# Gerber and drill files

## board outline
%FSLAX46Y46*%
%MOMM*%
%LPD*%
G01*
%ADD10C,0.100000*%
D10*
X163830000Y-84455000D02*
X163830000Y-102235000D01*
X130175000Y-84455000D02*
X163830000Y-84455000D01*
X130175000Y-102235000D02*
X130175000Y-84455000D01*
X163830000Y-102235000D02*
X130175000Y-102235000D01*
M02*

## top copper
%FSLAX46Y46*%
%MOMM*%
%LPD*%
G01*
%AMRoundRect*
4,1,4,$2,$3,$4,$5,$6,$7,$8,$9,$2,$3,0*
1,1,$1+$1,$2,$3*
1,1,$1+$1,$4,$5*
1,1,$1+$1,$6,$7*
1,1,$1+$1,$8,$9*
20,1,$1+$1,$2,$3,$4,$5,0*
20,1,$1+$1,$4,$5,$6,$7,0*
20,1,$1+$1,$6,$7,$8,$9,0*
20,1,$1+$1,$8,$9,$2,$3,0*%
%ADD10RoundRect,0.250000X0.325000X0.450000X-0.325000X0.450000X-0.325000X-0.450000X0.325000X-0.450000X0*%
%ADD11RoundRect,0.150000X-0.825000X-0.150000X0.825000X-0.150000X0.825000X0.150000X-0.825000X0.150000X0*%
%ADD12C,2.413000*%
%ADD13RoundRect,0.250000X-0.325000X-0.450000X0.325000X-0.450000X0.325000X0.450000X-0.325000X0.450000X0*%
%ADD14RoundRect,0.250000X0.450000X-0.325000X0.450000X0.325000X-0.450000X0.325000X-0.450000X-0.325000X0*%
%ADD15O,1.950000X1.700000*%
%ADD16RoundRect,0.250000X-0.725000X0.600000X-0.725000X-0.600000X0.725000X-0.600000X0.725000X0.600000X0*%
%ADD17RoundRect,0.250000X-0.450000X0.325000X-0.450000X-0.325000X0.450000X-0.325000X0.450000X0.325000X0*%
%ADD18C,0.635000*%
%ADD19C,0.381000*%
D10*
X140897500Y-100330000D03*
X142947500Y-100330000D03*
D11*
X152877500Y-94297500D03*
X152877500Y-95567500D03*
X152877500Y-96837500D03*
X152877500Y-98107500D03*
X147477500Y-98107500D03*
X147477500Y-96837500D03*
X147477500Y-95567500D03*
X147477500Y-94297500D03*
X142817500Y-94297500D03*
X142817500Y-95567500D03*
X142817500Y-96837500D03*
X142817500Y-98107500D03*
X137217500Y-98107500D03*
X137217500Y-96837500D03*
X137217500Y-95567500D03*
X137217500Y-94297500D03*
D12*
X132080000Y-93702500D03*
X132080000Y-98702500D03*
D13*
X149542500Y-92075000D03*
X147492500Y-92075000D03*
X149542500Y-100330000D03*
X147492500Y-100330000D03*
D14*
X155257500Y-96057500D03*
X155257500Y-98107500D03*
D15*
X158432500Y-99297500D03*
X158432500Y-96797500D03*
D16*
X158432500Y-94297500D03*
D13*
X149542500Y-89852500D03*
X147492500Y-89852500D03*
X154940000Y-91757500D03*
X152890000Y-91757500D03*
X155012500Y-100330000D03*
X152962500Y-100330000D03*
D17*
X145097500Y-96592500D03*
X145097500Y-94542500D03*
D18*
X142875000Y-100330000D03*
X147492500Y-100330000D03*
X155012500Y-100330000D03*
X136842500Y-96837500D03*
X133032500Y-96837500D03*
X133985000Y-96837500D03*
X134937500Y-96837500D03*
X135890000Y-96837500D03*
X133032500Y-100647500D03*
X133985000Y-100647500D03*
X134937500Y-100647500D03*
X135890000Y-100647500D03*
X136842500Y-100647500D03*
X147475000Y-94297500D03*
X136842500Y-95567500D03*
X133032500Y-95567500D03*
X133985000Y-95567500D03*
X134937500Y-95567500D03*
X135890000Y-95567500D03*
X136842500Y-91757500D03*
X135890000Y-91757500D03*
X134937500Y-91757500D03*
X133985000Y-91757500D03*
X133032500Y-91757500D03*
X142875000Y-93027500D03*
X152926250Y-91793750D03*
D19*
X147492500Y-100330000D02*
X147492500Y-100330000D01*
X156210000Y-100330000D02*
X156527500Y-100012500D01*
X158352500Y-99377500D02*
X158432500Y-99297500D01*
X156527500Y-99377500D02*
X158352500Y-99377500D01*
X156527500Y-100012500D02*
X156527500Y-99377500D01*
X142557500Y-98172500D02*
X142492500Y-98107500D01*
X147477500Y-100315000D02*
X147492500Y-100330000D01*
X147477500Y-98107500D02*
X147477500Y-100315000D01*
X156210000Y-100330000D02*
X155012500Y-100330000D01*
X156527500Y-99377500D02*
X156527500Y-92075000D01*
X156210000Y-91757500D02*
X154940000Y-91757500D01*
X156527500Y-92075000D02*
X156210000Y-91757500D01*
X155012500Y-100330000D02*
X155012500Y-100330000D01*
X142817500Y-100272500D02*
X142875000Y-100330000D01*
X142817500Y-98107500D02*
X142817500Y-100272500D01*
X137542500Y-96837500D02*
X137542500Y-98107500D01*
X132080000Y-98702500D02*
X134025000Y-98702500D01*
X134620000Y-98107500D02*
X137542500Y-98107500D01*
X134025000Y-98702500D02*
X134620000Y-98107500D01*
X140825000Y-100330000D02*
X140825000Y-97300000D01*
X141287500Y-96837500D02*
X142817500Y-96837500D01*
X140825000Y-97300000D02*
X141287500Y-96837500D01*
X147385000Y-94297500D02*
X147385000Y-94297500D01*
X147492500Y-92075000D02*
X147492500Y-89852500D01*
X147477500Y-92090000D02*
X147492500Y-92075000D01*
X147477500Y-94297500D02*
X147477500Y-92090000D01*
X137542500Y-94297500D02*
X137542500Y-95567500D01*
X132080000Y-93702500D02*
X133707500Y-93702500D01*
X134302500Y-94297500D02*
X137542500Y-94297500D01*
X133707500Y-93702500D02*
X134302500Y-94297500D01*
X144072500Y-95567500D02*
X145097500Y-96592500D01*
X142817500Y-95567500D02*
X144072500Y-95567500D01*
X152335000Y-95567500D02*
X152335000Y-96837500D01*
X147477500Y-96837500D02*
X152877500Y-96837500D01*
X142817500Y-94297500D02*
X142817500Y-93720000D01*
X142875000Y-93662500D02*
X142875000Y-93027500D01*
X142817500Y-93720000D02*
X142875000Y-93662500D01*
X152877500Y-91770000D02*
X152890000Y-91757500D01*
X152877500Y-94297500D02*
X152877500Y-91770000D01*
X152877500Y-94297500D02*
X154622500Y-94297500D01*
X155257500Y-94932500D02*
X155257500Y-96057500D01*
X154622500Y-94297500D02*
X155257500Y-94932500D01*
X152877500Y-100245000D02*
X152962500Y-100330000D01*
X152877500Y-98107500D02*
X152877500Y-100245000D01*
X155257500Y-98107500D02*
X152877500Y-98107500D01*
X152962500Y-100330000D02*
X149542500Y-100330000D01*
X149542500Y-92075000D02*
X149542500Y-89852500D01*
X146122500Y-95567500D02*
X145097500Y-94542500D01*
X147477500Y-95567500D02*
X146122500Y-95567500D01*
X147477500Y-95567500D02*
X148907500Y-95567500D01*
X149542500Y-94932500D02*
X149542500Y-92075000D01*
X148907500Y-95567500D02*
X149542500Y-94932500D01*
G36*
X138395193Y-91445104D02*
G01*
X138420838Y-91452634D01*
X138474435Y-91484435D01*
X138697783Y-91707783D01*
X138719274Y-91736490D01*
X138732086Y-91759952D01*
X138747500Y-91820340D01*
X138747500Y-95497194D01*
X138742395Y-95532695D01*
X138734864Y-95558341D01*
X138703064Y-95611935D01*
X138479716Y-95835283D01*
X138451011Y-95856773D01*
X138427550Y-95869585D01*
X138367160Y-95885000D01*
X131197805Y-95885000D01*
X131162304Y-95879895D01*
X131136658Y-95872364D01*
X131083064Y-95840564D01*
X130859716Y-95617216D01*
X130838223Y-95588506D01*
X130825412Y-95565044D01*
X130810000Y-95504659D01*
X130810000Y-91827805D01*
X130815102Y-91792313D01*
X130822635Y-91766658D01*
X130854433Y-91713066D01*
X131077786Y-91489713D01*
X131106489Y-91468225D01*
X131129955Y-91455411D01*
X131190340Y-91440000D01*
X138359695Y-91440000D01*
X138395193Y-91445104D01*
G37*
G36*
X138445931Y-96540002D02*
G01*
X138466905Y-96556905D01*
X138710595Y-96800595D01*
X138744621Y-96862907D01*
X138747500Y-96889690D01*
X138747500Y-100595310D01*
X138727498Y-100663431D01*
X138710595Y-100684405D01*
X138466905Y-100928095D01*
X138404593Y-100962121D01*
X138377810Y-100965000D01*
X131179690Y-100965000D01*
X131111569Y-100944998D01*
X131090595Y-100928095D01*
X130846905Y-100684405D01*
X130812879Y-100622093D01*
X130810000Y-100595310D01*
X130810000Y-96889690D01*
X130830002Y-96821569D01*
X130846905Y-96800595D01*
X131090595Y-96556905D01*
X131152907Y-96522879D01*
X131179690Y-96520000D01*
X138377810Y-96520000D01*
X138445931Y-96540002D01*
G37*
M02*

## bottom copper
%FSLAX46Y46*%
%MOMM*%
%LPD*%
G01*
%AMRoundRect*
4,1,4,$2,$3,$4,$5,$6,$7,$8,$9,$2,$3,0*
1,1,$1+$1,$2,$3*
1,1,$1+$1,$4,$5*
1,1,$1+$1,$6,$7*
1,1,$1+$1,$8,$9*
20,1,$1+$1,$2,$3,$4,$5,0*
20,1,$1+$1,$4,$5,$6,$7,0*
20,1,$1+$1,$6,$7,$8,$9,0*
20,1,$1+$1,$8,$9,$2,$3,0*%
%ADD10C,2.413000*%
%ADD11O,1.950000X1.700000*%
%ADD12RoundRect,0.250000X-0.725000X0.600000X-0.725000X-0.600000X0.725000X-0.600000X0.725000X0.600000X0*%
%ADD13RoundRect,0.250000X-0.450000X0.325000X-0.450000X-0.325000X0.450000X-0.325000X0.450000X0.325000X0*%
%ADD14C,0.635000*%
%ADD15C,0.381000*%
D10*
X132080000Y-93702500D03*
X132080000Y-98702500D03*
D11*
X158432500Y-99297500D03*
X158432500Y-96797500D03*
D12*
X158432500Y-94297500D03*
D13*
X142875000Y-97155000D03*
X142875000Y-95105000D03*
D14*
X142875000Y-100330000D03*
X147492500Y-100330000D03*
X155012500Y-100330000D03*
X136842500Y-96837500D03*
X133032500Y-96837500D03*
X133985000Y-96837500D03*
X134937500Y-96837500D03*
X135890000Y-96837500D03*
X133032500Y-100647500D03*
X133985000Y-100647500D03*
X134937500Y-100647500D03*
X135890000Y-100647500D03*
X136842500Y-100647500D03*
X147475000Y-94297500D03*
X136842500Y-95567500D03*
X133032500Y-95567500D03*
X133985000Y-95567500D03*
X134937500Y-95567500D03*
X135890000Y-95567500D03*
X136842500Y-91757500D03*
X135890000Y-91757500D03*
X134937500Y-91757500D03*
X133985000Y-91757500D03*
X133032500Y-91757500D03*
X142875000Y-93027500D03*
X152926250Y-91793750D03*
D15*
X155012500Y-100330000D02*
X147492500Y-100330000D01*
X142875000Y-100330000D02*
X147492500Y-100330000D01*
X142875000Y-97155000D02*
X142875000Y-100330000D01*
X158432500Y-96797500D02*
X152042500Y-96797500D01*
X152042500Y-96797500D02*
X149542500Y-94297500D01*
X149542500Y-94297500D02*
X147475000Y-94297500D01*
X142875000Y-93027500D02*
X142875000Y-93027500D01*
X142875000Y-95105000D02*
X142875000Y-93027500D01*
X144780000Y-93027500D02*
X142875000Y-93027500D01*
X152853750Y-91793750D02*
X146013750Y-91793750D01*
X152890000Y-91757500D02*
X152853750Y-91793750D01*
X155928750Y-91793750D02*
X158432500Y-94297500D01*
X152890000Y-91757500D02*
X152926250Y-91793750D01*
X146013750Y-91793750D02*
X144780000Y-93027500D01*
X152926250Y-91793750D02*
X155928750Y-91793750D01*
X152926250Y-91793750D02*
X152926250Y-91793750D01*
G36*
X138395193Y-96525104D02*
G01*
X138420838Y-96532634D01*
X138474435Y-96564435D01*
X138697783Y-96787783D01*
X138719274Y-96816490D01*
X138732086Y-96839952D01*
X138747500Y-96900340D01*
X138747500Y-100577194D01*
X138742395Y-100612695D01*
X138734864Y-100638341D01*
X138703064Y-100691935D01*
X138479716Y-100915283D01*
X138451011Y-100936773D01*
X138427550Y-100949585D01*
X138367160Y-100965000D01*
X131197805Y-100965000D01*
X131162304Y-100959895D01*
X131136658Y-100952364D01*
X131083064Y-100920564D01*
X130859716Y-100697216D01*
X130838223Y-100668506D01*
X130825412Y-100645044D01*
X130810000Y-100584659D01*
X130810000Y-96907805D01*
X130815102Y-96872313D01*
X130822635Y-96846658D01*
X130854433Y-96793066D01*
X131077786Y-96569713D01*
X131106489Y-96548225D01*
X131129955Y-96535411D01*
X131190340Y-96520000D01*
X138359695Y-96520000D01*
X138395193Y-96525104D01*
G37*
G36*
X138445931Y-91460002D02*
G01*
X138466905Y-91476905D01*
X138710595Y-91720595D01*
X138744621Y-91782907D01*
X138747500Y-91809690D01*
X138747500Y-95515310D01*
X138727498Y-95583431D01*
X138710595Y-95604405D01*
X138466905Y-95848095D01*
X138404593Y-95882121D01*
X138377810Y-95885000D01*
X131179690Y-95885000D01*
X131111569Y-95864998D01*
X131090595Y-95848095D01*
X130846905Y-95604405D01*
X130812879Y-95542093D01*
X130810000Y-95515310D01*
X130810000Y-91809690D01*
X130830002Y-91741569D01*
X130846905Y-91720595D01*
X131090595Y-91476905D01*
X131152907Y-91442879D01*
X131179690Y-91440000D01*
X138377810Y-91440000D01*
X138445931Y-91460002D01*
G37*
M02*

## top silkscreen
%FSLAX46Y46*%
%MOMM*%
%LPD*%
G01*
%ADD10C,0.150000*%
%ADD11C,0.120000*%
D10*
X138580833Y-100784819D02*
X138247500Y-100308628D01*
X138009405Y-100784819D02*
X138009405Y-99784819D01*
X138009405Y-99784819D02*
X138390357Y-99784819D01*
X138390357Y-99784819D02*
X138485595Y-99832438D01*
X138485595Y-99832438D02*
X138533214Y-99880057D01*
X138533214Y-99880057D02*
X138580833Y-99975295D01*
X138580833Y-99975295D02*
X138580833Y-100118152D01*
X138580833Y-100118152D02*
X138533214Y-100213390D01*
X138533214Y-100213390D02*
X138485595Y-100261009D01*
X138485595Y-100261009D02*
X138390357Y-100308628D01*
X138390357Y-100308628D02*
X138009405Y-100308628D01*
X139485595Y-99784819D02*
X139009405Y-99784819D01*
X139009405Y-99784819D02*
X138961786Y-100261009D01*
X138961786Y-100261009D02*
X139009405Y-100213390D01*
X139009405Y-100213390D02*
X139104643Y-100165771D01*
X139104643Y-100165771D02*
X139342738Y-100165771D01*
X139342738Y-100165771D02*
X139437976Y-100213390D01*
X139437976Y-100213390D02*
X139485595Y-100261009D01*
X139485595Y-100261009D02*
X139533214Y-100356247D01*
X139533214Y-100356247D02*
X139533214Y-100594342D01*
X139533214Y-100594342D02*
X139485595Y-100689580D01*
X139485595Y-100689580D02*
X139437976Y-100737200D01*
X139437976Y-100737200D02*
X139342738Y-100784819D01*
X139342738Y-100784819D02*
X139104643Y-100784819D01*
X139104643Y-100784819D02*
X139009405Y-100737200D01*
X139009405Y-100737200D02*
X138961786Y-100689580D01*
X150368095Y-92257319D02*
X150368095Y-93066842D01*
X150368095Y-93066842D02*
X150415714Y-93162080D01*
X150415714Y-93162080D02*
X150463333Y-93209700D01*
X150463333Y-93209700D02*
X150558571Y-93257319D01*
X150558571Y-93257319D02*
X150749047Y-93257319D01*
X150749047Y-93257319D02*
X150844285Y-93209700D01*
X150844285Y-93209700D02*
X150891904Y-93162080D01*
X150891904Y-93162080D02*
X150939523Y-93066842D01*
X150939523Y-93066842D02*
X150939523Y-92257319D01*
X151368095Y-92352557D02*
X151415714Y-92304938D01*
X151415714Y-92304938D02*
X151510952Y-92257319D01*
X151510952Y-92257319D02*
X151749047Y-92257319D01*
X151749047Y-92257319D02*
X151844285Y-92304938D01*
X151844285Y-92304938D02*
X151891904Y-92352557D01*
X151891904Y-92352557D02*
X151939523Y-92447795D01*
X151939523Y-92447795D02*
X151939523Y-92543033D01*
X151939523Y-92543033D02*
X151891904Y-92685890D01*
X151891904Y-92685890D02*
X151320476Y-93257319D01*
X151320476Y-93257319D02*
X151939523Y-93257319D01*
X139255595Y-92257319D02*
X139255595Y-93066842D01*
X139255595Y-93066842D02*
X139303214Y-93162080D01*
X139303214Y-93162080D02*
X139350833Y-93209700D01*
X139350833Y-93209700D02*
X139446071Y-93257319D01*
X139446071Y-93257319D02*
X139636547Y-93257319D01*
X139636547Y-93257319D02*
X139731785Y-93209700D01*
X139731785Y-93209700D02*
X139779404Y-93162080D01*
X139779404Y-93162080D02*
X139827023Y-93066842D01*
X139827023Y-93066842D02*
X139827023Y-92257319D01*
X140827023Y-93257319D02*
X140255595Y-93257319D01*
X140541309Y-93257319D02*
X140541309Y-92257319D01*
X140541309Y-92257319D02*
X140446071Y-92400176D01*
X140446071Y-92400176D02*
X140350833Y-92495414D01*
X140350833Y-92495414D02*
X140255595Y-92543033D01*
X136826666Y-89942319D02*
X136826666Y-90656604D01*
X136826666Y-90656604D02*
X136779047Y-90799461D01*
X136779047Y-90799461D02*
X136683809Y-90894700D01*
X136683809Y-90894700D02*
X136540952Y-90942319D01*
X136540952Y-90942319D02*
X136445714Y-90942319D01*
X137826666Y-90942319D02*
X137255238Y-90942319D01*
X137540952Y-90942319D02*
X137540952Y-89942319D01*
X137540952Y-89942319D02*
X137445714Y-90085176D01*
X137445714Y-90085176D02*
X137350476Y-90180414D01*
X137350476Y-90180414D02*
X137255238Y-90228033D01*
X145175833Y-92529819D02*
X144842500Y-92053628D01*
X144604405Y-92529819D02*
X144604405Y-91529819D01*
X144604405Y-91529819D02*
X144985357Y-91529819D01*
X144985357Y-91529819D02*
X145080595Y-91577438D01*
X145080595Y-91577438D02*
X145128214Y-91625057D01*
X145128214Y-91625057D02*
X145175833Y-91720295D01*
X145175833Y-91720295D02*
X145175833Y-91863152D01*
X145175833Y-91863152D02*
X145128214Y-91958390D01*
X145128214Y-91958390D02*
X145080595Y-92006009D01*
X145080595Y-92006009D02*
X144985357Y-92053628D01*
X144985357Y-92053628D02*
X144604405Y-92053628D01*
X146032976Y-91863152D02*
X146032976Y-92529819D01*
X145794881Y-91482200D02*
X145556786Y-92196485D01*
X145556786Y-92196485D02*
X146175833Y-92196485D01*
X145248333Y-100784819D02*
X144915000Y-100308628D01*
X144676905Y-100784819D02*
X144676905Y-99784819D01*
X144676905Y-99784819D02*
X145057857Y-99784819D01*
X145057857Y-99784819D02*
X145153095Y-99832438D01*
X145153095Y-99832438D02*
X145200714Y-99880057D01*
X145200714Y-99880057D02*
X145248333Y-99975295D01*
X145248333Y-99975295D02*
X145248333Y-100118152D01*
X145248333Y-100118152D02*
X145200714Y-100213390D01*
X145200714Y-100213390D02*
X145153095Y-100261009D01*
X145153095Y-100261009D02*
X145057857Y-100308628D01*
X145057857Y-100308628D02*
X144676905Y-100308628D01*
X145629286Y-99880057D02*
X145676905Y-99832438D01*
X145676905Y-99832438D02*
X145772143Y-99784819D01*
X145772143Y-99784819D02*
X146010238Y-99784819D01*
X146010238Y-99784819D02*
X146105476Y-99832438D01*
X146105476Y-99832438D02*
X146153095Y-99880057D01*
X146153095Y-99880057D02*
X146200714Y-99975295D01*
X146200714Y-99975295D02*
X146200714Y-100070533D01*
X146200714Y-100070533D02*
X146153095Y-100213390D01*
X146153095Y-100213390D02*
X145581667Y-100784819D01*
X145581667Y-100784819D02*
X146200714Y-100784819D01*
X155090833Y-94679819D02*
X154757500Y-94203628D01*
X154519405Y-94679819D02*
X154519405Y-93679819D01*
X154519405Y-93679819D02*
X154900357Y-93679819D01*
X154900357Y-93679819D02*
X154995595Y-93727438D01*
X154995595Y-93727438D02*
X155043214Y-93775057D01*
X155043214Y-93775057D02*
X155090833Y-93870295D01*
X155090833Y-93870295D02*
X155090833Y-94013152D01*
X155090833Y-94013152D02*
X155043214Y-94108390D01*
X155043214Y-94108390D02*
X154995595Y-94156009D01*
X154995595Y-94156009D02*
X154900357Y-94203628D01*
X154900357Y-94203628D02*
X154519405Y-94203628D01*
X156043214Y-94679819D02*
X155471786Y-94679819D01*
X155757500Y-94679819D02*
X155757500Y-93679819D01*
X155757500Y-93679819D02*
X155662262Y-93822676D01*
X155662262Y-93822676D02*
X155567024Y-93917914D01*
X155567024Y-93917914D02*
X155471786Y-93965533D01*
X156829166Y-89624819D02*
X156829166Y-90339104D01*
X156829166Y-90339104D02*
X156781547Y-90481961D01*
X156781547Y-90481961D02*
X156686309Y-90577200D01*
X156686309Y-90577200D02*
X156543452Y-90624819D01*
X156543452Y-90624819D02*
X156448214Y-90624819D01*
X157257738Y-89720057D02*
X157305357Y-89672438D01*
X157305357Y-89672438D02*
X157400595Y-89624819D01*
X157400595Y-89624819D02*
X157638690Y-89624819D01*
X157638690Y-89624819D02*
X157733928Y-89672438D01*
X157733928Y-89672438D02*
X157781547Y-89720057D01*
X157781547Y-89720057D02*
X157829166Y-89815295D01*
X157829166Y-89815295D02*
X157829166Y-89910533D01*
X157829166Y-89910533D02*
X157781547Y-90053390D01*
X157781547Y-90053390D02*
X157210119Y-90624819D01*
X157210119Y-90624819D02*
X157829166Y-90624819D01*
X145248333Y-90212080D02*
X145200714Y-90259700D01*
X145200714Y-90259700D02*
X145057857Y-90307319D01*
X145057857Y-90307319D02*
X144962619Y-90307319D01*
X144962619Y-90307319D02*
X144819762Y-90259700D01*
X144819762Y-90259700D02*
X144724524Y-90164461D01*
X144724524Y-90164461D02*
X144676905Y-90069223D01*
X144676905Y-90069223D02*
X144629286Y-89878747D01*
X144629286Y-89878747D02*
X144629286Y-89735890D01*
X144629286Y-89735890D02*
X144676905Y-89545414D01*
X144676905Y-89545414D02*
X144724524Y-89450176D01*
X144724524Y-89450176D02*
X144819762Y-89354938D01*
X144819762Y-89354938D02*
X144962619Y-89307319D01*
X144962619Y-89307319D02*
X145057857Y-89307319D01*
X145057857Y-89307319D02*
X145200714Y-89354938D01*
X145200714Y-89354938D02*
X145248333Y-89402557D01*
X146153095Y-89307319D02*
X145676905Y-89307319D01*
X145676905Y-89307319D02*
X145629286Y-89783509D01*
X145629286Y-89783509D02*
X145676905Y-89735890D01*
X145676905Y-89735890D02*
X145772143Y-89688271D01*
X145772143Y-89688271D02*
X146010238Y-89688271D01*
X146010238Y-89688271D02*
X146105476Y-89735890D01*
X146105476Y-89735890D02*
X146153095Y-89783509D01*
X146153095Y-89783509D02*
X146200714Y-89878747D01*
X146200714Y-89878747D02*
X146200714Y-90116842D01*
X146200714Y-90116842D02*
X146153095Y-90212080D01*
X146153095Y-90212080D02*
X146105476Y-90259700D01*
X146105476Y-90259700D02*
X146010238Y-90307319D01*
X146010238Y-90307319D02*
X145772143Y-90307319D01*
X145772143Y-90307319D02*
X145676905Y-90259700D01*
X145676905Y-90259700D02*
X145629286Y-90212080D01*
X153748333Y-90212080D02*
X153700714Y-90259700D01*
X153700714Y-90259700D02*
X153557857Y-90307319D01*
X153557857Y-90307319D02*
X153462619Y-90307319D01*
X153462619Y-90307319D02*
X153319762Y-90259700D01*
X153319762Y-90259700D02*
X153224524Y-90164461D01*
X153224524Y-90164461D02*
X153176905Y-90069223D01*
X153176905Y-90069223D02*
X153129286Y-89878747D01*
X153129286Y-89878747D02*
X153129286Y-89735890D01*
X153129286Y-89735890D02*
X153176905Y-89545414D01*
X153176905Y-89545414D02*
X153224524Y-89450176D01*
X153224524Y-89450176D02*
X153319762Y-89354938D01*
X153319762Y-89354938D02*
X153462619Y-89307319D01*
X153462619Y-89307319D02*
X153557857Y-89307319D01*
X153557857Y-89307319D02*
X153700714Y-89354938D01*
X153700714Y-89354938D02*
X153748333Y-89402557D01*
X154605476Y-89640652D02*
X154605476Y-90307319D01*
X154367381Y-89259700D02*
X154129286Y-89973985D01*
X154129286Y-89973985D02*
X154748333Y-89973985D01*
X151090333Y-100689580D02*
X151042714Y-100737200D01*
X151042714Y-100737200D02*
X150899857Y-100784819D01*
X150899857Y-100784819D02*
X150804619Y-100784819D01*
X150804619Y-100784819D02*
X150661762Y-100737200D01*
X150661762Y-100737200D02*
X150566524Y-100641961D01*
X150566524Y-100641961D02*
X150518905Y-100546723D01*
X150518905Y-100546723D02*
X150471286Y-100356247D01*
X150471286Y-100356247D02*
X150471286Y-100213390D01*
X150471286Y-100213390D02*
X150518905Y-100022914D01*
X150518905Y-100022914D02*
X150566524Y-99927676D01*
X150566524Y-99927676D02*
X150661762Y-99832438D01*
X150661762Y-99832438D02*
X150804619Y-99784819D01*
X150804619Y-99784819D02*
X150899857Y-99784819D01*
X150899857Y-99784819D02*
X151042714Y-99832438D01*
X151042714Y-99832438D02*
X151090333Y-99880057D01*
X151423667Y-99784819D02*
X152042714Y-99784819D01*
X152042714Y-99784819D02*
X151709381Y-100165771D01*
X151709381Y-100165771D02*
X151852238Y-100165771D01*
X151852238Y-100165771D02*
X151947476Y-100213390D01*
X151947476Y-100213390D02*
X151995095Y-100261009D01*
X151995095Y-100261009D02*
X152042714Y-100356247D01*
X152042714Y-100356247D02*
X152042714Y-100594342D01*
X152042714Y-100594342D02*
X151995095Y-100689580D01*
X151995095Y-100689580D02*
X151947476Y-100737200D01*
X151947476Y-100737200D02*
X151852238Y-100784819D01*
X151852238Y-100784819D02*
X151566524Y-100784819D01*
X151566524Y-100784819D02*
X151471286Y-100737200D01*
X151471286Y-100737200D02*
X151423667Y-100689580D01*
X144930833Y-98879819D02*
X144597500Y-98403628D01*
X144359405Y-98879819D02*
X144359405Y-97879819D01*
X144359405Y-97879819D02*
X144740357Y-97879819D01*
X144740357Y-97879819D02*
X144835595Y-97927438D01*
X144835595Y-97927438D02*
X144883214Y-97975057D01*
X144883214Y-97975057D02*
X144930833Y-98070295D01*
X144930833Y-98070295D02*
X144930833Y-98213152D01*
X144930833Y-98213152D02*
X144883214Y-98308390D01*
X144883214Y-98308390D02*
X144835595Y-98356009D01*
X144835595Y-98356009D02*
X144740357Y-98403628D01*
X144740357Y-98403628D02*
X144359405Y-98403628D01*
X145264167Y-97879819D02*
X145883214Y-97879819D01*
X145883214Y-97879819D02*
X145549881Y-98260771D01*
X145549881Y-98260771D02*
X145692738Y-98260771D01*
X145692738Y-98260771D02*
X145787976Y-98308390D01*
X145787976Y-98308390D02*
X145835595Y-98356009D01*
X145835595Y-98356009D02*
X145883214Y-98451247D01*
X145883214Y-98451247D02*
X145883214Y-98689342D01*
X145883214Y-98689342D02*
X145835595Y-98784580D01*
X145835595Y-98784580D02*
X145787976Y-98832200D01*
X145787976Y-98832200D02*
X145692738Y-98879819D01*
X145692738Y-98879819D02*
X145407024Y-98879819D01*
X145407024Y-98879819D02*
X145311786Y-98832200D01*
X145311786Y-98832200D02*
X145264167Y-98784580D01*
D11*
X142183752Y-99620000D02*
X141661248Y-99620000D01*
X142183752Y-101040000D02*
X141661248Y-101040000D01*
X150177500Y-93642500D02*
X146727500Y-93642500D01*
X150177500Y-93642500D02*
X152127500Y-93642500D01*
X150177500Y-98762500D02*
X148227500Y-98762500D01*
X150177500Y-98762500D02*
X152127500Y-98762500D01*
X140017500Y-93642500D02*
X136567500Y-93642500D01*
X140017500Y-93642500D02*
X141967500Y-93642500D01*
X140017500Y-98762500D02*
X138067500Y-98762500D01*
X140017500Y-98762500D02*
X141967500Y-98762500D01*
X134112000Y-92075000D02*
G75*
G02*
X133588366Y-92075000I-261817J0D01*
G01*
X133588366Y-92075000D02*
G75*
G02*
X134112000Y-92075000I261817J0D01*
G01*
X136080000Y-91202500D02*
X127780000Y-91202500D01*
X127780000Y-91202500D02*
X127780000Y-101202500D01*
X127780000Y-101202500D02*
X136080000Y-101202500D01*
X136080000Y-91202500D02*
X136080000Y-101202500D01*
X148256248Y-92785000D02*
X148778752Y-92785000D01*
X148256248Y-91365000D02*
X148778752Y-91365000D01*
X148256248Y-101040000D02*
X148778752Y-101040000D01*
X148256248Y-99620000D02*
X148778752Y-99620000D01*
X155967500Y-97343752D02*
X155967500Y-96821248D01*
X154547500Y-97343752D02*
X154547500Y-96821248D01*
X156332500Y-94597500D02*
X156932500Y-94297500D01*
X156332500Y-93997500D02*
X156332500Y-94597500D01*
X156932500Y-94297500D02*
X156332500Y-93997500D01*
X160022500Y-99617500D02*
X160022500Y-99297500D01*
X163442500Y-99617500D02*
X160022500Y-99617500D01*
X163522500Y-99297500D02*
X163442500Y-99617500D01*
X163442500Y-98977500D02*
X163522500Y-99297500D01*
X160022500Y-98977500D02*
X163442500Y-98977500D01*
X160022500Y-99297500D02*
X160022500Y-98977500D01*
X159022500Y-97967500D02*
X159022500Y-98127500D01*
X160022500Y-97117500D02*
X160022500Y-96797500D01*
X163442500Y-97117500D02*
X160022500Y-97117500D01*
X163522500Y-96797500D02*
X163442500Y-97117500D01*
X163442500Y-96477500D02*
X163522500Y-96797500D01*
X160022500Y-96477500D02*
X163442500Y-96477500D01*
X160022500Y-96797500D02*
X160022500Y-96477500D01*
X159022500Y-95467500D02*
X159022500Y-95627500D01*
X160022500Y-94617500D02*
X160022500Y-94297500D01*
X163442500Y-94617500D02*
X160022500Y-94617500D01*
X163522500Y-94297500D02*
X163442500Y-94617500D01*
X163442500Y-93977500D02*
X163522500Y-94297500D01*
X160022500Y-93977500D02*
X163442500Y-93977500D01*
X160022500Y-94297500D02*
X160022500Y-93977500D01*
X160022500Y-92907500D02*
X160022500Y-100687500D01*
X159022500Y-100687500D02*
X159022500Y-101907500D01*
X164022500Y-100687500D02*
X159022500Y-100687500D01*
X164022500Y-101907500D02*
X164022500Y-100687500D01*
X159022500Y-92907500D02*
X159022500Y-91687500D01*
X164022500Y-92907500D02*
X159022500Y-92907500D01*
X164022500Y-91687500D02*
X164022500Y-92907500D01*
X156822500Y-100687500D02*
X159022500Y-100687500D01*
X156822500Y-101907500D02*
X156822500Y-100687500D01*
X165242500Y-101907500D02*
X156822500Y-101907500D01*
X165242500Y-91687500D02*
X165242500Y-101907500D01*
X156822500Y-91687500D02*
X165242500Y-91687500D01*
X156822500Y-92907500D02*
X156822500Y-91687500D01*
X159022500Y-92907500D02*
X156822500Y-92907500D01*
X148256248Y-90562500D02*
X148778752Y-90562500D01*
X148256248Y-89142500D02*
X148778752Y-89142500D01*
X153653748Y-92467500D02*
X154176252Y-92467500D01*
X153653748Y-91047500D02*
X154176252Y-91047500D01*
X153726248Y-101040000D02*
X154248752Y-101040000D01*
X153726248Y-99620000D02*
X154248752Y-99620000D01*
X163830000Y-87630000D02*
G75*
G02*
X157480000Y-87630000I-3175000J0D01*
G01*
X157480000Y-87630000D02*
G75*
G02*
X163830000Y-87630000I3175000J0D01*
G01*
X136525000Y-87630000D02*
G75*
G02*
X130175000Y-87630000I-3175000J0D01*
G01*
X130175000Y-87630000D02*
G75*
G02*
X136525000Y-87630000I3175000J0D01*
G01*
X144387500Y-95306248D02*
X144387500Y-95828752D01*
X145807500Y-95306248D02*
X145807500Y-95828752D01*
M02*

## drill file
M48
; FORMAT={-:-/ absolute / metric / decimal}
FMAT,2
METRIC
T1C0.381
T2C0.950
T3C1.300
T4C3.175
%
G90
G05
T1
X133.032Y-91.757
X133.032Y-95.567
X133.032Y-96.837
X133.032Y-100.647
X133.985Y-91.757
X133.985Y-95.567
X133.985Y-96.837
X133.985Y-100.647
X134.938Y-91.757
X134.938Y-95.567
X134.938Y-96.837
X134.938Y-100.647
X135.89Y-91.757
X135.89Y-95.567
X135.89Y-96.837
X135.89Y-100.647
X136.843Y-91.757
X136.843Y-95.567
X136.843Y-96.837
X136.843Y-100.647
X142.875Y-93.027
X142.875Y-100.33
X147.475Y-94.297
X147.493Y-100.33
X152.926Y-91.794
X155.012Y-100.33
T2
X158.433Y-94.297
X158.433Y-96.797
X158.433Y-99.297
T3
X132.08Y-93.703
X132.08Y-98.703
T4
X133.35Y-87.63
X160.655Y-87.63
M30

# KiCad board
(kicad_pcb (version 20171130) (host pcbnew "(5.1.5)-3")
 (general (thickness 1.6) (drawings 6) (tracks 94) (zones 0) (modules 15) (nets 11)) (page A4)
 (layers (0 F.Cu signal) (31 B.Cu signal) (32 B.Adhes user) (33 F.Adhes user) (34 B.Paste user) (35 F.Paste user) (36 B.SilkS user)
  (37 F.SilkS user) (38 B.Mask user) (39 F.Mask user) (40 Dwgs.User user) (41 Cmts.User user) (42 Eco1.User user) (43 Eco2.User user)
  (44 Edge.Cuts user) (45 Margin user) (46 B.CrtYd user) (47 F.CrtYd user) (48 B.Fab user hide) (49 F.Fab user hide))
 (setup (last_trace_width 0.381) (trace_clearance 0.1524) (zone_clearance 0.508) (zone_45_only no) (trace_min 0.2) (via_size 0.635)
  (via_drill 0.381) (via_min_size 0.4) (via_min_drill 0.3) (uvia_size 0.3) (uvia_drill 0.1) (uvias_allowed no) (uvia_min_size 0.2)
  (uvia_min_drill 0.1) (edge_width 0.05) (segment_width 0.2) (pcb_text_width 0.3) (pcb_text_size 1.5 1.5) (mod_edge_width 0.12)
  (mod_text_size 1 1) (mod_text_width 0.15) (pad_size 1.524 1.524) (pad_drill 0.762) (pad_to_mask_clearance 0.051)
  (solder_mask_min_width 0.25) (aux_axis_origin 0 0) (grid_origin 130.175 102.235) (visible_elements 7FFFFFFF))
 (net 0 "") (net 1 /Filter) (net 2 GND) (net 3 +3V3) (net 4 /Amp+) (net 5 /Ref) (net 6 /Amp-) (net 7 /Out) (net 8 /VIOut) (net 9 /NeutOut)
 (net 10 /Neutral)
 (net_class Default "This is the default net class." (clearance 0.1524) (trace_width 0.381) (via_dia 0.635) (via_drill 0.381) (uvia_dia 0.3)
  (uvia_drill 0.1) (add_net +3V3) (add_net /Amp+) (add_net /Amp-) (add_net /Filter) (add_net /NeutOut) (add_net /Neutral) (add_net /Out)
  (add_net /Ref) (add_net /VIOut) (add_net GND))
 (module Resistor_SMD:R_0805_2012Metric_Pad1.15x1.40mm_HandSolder (layer F.Cu) (at 141.9225 100.33 180)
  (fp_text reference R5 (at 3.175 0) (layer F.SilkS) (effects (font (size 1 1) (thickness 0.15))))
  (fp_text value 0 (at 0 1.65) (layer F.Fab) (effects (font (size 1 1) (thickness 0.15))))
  (fp_line (start -0.261252 0.71) (end 0.261252 0.71) (layer F.SilkS) (width 0.12))
  (fp_line (start -0.261252 -0.71) (end 0.261252 -0.71) (layer F.SilkS) (width 0.12))
  (pad 2 smd roundrect (at 1.025 0 180) (size 1.15 1.4) (layers F.Cu F.Paste F.Mask) (roundrect_rratio 0.217391) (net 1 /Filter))
  (pad 1 smd roundrect (at -1.025 0 180) (size 1.15 1.4) (layers F.Cu F.Paste F.Mask) (roundrect_rratio 0.217391) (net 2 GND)))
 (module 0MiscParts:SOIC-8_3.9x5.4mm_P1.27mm (layer F.Cu) (at 150.1775 96.2025)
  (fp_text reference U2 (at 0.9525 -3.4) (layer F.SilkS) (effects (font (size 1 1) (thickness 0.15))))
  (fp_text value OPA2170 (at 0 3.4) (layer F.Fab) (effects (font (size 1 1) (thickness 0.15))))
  (fp_line (start 0 -2.56) (end -3.45 -2.56) (layer F.SilkS) (width 0.12))
  (fp_line (start 0 -2.56) (end 1.95 -2.56) (layer F.SilkS) (width 0.12))
  (fp_line (start 0 2.56) (end -1.95 2.56) (layer F.SilkS) (width 0.12))
  (fp_line (start 0 2.56) (end 1.95 2.56) (layer F.SilkS) (width 0.12))
  (pad 8 smd roundrect (at 2.7 -1.905) (size 1.95 0.6) (layers F.Cu F.Paste F.Mask) (roundrect_rratio 0.25) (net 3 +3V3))
  (pad 7 smd roundrect (at 2.7 -0.635) (size 1.95 0.6) (layers F.Cu F.Paste F.Mask) (roundrect_rratio 0.25) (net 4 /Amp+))
  (pad 6 smd roundrect (at 2.7 0.635) (size 1.95 0.6) (layers F.Cu F.Paste F.Mask) (roundrect_rratio 0.25) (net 4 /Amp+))
  (pad 5 smd roundrect (at 2.7 1.905) (size 1.95 0.6) (layers F.Cu F.Paste F.Mask) (roundrect_rratio 0.25) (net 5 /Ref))
  (pad 4 smd roundrect (at -2.7 1.905) (size 1.95 0.6) (layers F.Cu F.Paste F.Mask) (roundrect_rratio 0.25) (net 2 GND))
  (pad 3 smd roundrect (at -2.7 0.635) (size 1.95 0.6) (layers F.Cu F.Paste F.Mask) (roundrect_rratio 0.25) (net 4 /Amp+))
  (pad 2 smd roundrect (at -2.7 -0.635) (size 1.95 0.6) (layers F.Cu F.Paste F.Mask) (roundrect_rratio 0.25) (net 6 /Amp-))
  (pad 1 smd roundrect (at -2.7 -1.905) (size 1.95 0.6) (layers F.Cu F.Paste F.Mask) (roundrect_rratio 0.25) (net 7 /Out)))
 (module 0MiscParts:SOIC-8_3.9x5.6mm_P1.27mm (layer F.Cu) (at 140.0175 96.2025)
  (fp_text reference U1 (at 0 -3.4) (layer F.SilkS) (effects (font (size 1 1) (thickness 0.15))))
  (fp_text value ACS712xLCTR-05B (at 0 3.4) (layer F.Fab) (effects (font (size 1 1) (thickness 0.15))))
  (fp_line (start 0 -2.56) (end -3.45 -2.56) (layer F.SilkS) (width 0.12))
  (fp_line (start 0 -2.56) (end 1.95 -2.56) (layer F.SilkS) (width 0.12))
  (fp_line (start 0 2.56) (end -1.95 2.56) (layer F.SilkS) (width 0.12))
  (fp_line (start 0 2.56) (end 1.95 2.56) (layer F.SilkS) (width 0.12))
  (pad 8 smd roundrect (at 2.8 -1.905) (size 1.95 0.6) (layers F.Cu F.Paste F.Mask) (roundrect_rratio 0.25) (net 3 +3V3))
  (pad 7 smd roundrect (at 2.8 -0.635) (size 1.95 0.6) (layers F.Cu F.Paste F.Mask) (roundrect_rratio 0.25) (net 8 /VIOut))
  (pad 6 smd roundrect (at 2.8 0.635) (size 1.95 0.6) (layers F.Cu F.Paste F.Mask) (roundrect_rratio 0.25) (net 1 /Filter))
  (pad 5 smd roundrect (at 2.8 1.905) (size 1.95 0.6) (layers F.Cu F.Paste F.Mask) (roundrect_rratio 0.25) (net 2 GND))
  (pad 4 smd roundrect (at -2.8 1.905) (size 1.95 0.6) (layers F.Cu F.Paste F.Mask) (roundrect_rratio 0.25) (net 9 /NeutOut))
  (pad 3 smd roundrect (at -2.8 0.635) (size 1.95 0.6) (layers F.Cu F.Paste F.Mask) (roundrect_rratio 0.25) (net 9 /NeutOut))
  (pad 2 smd roundrect (at -2.8 -0.635) (size 1.95 0.6) (layers F.Cu F.Paste F.Mask) (roundrect_rratio 0.25) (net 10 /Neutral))
  (pad 1 smd roundrect (at -2.8 -1.905) (size 1.95 0.6) (layers F.Cu F.Paste F.Mask) (roundrect_rratio 0.25) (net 10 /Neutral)))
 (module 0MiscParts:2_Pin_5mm (layer F.Cu) (at 132.08 96.2025 270)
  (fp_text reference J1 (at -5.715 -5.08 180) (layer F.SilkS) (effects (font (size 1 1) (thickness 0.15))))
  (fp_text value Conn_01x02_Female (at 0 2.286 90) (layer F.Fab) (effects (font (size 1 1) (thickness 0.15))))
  (fp_circle (center -4.1275 -1.770183) (end -4.064 -1.516183) (layer F.SilkS) (width 0.12))
  (fp_line (start -5 -4) (end -5 4.3) (layer F.SilkS) (width 0.12))
  (fp_line (start -5 4.3) (end 5 4.3) (layer F.SilkS) (width 0.12))
  (fp_line (start 5 4.3) (end 5 -4) (layer F.SilkS) (width 0.12))
  (fp_line (start -5 -4) (end 5 -4) (layer F.SilkS) (width 0.12))
  (pad 1 thru_hole circle (at -2.5 0 270) (size 2.413 2.413) (drill 1.3) (layers *.Cu *.Mask) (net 10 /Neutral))
  (pad 2 thru_hole circle (at 2.5 0 270) (size 2.413 2.413) (drill 1.3) (layers *.Cu *.Mask) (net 9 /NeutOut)))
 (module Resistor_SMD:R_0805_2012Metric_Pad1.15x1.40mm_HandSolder (layer F.Cu) (at 148.5175 92.075)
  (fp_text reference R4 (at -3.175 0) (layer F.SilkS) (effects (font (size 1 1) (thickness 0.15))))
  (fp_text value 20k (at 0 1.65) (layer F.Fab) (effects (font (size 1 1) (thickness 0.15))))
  (fp_line (start -0.261252 0.71) (end 0.261252 0.71) (layer F.SilkS) (width 0.12))
  (fp_line (start -0.261252 -0.71) (end 0.261252 -0.71) (layer F.SilkS) (width 0.12))
  (pad 2 smd roundrect (at 1.025 0) (size 1.15 1.4) (layers F.Cu F.Paste F.Mask) (roundrect_rratio 0.217391) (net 6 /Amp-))
  (pad 1 smd roundrect (at -1.025 0) (size 1.15 1.4) (layers F.Cu F.Paste F.Mask) (roundrect_rratio 0.217391) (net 7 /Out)))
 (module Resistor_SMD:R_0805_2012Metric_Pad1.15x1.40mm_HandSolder (layer F.Cu) (at 148.5175 100.33)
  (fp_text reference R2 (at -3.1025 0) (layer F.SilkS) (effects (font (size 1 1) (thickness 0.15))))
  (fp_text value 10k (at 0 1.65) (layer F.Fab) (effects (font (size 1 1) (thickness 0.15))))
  (fp_line (start -0.261252 0.71) (end 0.261252 0.71) (layer F.SilkS) (width 0.12))
  (fp_line (start -0.261252 -0.71) (end 0.261252 -0.71) (layer F.SilkS) (width 0.12))
  (pad 2 smd roundrect (at 1.025 0) (size 1.15 1.4) (layers F.Cu F.Paste F.Mask) (roundrect_rratio 0.217391) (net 5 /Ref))
  (pad 1 smd roundrect (at -1.025 0) (size 1.15 1.4) (layers F.Cu F.Paste F.Mask) (roundrect_rratio 0.217391) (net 2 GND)))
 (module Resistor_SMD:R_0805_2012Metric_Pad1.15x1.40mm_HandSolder (layer F.Cu) (at 155.2575 97.0825 90)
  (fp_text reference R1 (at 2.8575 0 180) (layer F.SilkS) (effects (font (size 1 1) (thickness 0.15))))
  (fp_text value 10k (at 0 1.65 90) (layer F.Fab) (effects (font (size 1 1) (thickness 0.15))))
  (fp_line (start -0.261252 0.71) (end 0.261252 0.71) (layer F.SilkS) (width 0.12))
  (fp_line (start -0.261252 -0.71) (end 0.261252 -0.71) (layer F.SilkS) (width 0.12))
  (pad 2 smd roundrect (at 1.025 0 90) (size 1.15 1.4) (layers F.Cu F.Paste F.Mask) (roundrect_rratio 0.217391) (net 3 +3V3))
  (pad 1 smd roundrect (at -1.025 0 90) (size 1.15 1.4) (layers F.Cu F.Paste F.Mask) (roundrect_rratio 0.217391) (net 5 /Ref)))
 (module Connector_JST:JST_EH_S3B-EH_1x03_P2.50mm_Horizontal (layer F.Cu) (at 158.4325 94.2975 270)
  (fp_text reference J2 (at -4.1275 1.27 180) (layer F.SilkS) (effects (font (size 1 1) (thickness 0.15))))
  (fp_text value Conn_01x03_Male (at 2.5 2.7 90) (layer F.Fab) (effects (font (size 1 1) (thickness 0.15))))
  (fp_line (start 0.3 2.1) (end 0 1.5) (layer F.SilkS) (width 0.12))
  (fp_line (start -0.3 2.1) (end 0.3 2.1) (layer F.SilkS) (width 0.12))
  (fp_line (start 0 1.5) (end -0.3 2.1) (layer F.SilkS) (width 0.12))
  (fp_line (start 5.32 -1.59) (end 5 -1.59) (layer F.SilkS) (width 0.12))
  (fp_line (start 5.32 -5.01) (end 5.32 -1.59) (layer F.SilkS) (width 0.12))
  (fp_line (start 5 -5.09) (end 5.32 -5.01) (layer F.SilkS) (width 0.12))
  (fp_line (start 4.68 -5.01) (end 5 -5.09) (layer F.SilkS) (width 0.12))
  (fp_line (start 4.68 -1.59) (end 4.68 -5.01) (layer F.SilkS) (width 0.12))
  (fp_line (start 5 -1.59) (end 4.68 -1.59) (layer F.SilkS) (width 0.12))
  (fp_line (start 3.67 -0.59) (end 3.83 -0.59) (layer F.SilkS) (width 0.12))
  (fp_line (start 2.82 -1.59) (end 2.5 -1.59) (layer F.SilkS) (width 0.12))
  (fp_line (start 2.82 -5.01) (end 2.82 -1.59) (layer F.SilkS) (width 0.12))
  (fp_line (start 2.5 -5.09) (end 2.82 -5.01) (layer F.SilkS) (width 0.12))
  (fp_line (start 2.18 -5.01) (end 2.5 -5.09) (layer F.SilkS) (width 0.12))
  (fp_line (start 2.18 -1.59) (end 2.18 -5.01) (layer F.SilkS) (width 0.12))
  (fp_line (start 2.5 -1.59) (end 2.18 -1.59) (layer F.SilkS) (width 0.12))
  (fp_line (start 1.17 -0.59) (end 1.33 -0.59) (layer F.SilkS) (width 0.12))
  (fp_line (start 0.32 -1.59) (end 0 -1.59) (layer F.SilkS) (width 0.12))
  (fp_line (start 0.32 -5.01) (end 0.32 -1.59) (layer F.SilkS) (width 0.12))
  (fp_line (start 0 -5.09) (end 0.32 -5.01) (layer F.SilkS) (width 0.12))
  (fp_line (start -0.32 -5.01) (end 0 -5.09) (layer F.SilkS) (width 0.12))
  (fp_line (start -0.32 -1.59) (end -0.32 -5.01) (layer F.SilkS) (width 0.12))
  (fp_line (start 0 -1.59) (end -0.32 -1.59) (layer F.SilkS) (width 0.12))
  (fp_line (start -1.39 -1.59) (end 6.39 -1.59) (layer F.SilkS) (width 0.12))
  (fp_line (start 6.39 -0.59) (end 7.61 -0.59) (layer F.SilkS) (width 0.12))
  (fp_line (start 6.39 -5.59) (end 6.39 -0.59) (layer F.SilkS) (width 0.12))
  (fp_line (start 7.61 -5.59) (end 6.39 -5.59) (layer F.SilkS) (width 0.12))
  (fp_line (start -1.39 -0.59) (end -2.61 -0.59) (layer F.SilkS) (width 0.12))
  (fp_line (start -1.39 -5.59) (end -1.39 -0.59) (layer F.SilkS) (width 0.12))
  (fp_line (start -2.61 -5.59) (end -1.39 -5.59) (layer F.SilkS) (width 0.12))
  (fp_line (start 6.39 1.61) (end 6.39 -0.59) (layer F.SilkS) (width 0.12))
  (fp_line (start 7.61 1.61) (end 6.39 1.61) (layer F.SilkS) (width 0.12))
  (fp_line (start 7.61 -6.81) (end 7.61 1.61) (layer F.SilkS) (width 0.12))
  (fp_line (start -2.61 -6.81) (end 7.61 -6.81) (layer F.SilkS) (width 0.12))
  (fp_line (start -2.61 1.61) (end -2.61 -6.81) (layer F.SilkS) (width 0.12))
  (fp_line (start -1.39 1.61) (end -2.61 1.61) (layer F.SilkS) (width 0.12))
  (fp_line (start -1.39 -0.59) (end -1.39 1.61) (layer F.SilkS) (width 0.12))
  (pad 3 thru_hole oval (at 5 0 270) (size 1.7 1.95) (drill 0.95) (layers *.Cu *.Mask) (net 2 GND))
  (pad 2 thru_hole oval (at 2.5 0 270) (size 1.7 1.95) (drill 0.95) (layers *.Cu *.Mask) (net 7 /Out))
  (pad 1 thru_hole roundrect (at 0 0 270) (size 1.7 1.95) (drill 0.95) (layers *.Cu *.Mask) (roundrect_rratio 0.147059) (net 3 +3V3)))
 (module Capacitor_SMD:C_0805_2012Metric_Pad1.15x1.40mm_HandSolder (layer F.Cu) (at 148.5175 89.8525)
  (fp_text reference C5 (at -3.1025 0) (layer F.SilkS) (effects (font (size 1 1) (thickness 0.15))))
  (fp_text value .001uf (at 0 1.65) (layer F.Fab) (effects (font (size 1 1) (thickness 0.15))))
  (fp_line (start -0.261252 0.71) (end 0.261252 0.71) (layer F.SilkS) (width 0.12))
  (fp_line (start -0.261252 -0.71) (end 0.261252 -0.71) (layer F.SilkS) (width 0.12))
  (pad 2 smd roundrect (at 1.025 0) (size 1.15 1.4) (layers F.Cu F.Paste F.Mask) (roundrect_rratio 0.217391) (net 6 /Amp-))
  (pad 1 smd roundrect (at -1.025 0) (size 1.15 1.4) (layers F.Cu F.Paste F.Mask) (roundrect_rratio 0.217391) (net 7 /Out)))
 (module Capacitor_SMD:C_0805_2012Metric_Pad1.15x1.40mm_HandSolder (layer F.Cu) (at 153.915 91.7575)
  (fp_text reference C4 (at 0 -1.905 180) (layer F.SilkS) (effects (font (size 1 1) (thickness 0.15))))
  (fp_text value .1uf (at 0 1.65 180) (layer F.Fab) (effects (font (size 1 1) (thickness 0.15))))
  (fp_line (start -0.261252 0.71) (end 0.261252 0.71) (layer F.SilkS) (width 0.12))
  (fp_line (start -0.261252 -0.71) (end 0.261252 -0.71) (layer F.SilkS) (width 0.12))
  (pad 2 smd roundrect (at 1.025 0) (size 1.15 1.4) (layers F.Cu F.Paste F.Mask) (roundrect_rratio 0.217391) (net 2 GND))
  (pad 1 smd roundrect (at -1.025 0) (size 1.15 1.4) (layers F.Cu F.Paste F.Mask) (roundrect_rratio 0.217391) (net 3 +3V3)))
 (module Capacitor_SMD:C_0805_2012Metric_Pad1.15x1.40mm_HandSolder (layer F.Cu) (at 153.9875 100.33)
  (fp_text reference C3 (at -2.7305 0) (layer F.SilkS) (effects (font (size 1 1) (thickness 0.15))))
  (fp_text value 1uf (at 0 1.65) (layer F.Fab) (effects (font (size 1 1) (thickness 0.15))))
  (fp_line (start -0.261252 0.71) (end 0.261252 0.71) (layer F.SilkS) (width 0.12))
  (fp_line (start -0.261252 -0.71) (end 0.261252 -0.71) (layer F.SilkS) (width 0.12))
  (pad 2 smd roundrect (at 1.025 0) (size 1.15 1.4) (layers F.Cu F.Paste F.Mask) (roundrect_rratio 0.217391) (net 2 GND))
  (pad 1 smd roundrect (at -1.025 0) (size 1.15 1.4) (layers F.Cu F.Paste F.Mask) (roundrect_rratio 0.217391) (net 5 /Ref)))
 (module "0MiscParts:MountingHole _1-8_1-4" (layer F.Cu) (at 160.655 87.63)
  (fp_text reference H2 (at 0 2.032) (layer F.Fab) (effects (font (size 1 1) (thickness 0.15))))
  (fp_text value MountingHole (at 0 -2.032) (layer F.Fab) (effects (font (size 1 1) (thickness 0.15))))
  (fp_circle (center 0 0) (end 3.175 0) (layer F.SilkS) (width 0.12))
  (pad "" np_thru_hole circle (at 0 0) (size 3.175 3.175) (drill 3.175) (layers *.Cu *.Mask)))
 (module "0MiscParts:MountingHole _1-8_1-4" (layer F.Cu) (at 133.35 87.63)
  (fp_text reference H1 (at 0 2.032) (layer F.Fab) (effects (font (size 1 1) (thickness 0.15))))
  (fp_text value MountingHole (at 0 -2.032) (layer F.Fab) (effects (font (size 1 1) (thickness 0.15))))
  (fp_circle (center 0 0) (end 3.175 0) (layer F.SilkS) (width 0.12))
  (pad "" np_thru_hole circle (at 0 0) (size 3.175 3.175) (drill 3.175) (layers *.Cu *.Mask)))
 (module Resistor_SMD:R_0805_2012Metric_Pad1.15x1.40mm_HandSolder (layer F.Cu) (at 145.0975 95.5675 270)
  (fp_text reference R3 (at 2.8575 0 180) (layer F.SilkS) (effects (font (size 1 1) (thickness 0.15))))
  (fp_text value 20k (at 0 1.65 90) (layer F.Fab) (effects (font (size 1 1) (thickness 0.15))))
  (fp_line (start -0.261252 0.71) (end 0.261252 0.71) (layer F.SilkS) (width 0.12))
  (fp_line (start -0.261252 -0.71) (end 0.261252 -0.71) (layer F.SilkS) (width 0.12))
  (pad 2 smd roundrect (at 1.025 0 270) (size 1.15 1.4) (layers F.Cu F.Paste F.Mask) (roundrect_rratio 0.217391) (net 8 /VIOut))
  (pad 1 smd roundrect (at -1.025 0 270) (size 1.15 1.4) (layers F.Cu F.Paste F.Mask) (roundrect_rratio 0.217391) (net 6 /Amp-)))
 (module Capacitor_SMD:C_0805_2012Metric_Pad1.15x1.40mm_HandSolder (layer B.Cu) (at 142.875 96.13 270)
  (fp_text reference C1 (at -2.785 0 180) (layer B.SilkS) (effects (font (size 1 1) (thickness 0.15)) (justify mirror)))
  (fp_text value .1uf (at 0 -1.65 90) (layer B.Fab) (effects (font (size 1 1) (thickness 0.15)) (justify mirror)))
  (pad 2 smd roundrect (at 1.025 0 270) (size 1.15 1.4) (layers B.Cu B.Paste B.Mask) (roundrect_rratio 0.217391) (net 2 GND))
  (pad 1 smd roundrect (at -1.025 0 270) (size 1.15 1.4) (layers B.Cu B.Paste B.Mask) (roundrect_rratio 0.217391) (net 3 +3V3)))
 (gr_line (start 163.83 84.455) (end 163.83 102.235) (layer Edge.Cuts) (width 0.1))
 (gr_line (start 130.175 84.455) (end 163.83 84.455) (layer Edge.Cuts) (width 0.1))
 (gr_line (start 130.175 102.235) (end 130.175 84.455) (layer Edge.Cuts) (width 0.1))
 (gr_line (start 163.83 102.235) (end 130.175 102.235) (layer Edge.Cuts) (width 0.1))
 (via (at 142.875 100.33) (size 0.635) (drill 0.381) (layers F.Cu B.Cu) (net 2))
 (segment (start 147.4925 100.33) (end 147.4925 100.33) (width 0.381) (layer F.Cu) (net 2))
 (via (at 147.4925 100.33) (size 0.635) (drill 0.381) (layers F.Cu B.Cu) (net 2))
 (segment (start 156.21 100.33) (end 156.5275 100.0125) (width 0.381) (layer F.Cu) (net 2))
 (segment (start 158.3525 99.3775) (end 158.4325 99.2975) (width 0.381) (layer F.Cu) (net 2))
 (segment (start 156.5275 99.3775) (end 158.3525 99.3775) (width 0.381) (layer F.Cu) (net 2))
 (segment (start 156.5275 100.0125) (end 156.5275 99.3775) (width 0.381) (layer F.Cu) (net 2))
 (segment (start 142.5575 98.1725) (end 142.4925 98.1075) (width 0.381) (layer F.Cu) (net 2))
 (segment (start 147.4775 100.315) (end 147.4925 100.33) (width 0.381) (layer F.Cu) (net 2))
 (segment (start 147.4775 98.1075) (end 147.4775 100.315) (width 0.381) (layer F.Cu) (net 2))
 (segment (start 156.21 100.33) (end 155.0125 100.33) (width 0.381) (layer F.Cu) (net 2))
 (segment (start 156.5275 99.3775) (end 156.5275 92.075) (width 0.381) (layer F.Cu) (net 2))
 (segment (start 156.21 91.7575) (end 154.94 91.7575) (width 0.381) (layer F.Cu) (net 2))
 (segment (start 156.5275 92.075) (end 156.21 91.7575) (width 0.381) (layer F.Cu) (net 2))
 (segment (start 155.0125 100.33) (end 155.0125 100.33) (width 0.381) (layer F.Cu) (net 2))
 (via (at 155.0125 100.33) (size 0.635) (drill 0.381) (layers F.Cu B.Cu) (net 2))
 (segment (start 155.0125 100.33) (end 147.4925 100.33) (width 0.381) (layer B.Cu) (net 2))
 (segment (start 142.8175 100.2725) (end 142.875 100.33) (width 0.381) (layer F.Cu) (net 2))
 (segment (start 142.8175 98.1075) (end 142.8175 100.2725) (width 0.381) (layer F.Cu) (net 2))
 (segment (start 142.875 100.33) (end 147.4925 100.33) (width 0.381) (layer B.Cu) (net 2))
 (segment (start 142.875 97.155) (end 142.875 100.33) (width 0.381) (layer B.Cu) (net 2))
 (via (at 136.8425 96.8375) (size 0.635) (drill 0.381) (layers F.Cu B.Cu) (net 9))
 (segment (start 137.5425 96.8375) (end 137.5425 98.1075) (width 0.381) (layer F.Cu) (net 9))
 (segment (start 132.08 98.7025) (end 134.025 98.7025) (width 0.381) (layer F.Cu) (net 9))
 (segment (start 134.62 98.1075) (end 137.5425 98.1075) (width 0.381) (layer F.Cu) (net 9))
 (segment (start 134.025 98.7025) (end 134.62 98.1075) (width 0.381) (layer F.Cu) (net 9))
 (via (at 133.0325 96.8375) (size 0.635) (drill 0.381) (layers F.Cu B.Cu) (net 9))
 (via (at 133.985 96.8375) (size 0.635) (drill 0.381) (layers F.Cu B.Cu) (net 9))
 (via (at 134.9375 96.8375) (size 0.635) (drill 0.381) (layers F.Cu B.Cu) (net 9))
 (via (at 135.89 96.8375) (size 0.635) (drill 0.381) (layers F.Cu B.Cu) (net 9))
 (via (at 133.0325 100.6475) (size 0.635) (drill 0.381) (layers F.Cu B.Cu) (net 9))
 (via (at 133.985 100.6475) (size 0.635) (drill 0.381) (layers F.Cu B.Cu) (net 9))
 (via (at 134.9375 100.6475) (size 0.635) (drill 0.381) (layers F.Cu B.Cu) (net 9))
 (via (at 135.89 100.6475) (size 0.635) (drill 0.381) (layers F.Cu B.Cu) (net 9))
 (via (at 136.8425 100.6475) (size 0.635) (drill 0.381) (layers F.Cu B.Cu) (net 9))
 (segment (start 140.825 100.33) (end 140.825 97.3) (width 0.381) (layer F.Cu) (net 1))
 (segment (start 141.2875 96.8375) (end 142.8175 96.8375) (width 0.381) (layer F.Cu) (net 1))
 (segment (start 140.825 97.3) (end 141.2875 96.8375) (width 0.381) (layer F.Cu) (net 1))
 (segment (start 147.385 94.2975) (end 147.385 94.2975) (width 0.381) (layer F.Cu) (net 7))
 (via (at 147.475 94.2975) (size 0.635) (drill 0.381) (layers F.Cu B.Cu) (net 7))
 (segment (start 158.4325 96.7975) (end 152.0425 96.7975) (width 0.381) (layer B.Cu) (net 7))
 (segment (start 152.0425 96.7975) (end 149.5425 94.2975) (width 0.381) (layer B.Cu) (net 7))
 (segment (start 147.4925 92.075) (end 147.4925 89.8525) (width 0.381) (layer F.Cu) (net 7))
 (segment (start 147.4775 92.09) (end 147.4925 92.075) (width 0.381) (layer F.Cu) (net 7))
 (segment (start 147.4775 94.2975) (end 147.4775 92.09) (width 0.381) (layer F.Cu) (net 7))
 (segment (start 149.5425 94.2975) (end 147.475 94.2975) (width 0.381) (layer B.Cu) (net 7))
 (via (at 136.8425 95.5675) (size 0.635) (drill 0.381) (layers F.Cu B.Cu) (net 10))
 (segment (start 137.5425 94.2975) (end 137.5425 95.5675) (width 0.381) (layer F.Cu) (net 10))
 (segment (start 132.08 93.7025) (end 133.7075 93.7025) (width 0.381) (layer F.Cu) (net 10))
 (segment (start 134.3025 94.2975) (end 137.5425 94.2975) (width 0.381) (layer F.Cu) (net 10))
 (segment (start 133.7075 93.7025) (end 134.3025 94.2975) (width 0.381) (layer F.Cu) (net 10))
 (via (at 133.0325 95.5675) (size 0.635) (drill 0.381) (layers F.Cu B.Cu) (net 10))
 (via (at 133.985 95.5675) (size 0.635) (drill 0.381) (layers F.Cu B.Cu) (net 10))
 (via (at 134.9375 95.5675) (size 0.635) (drill 0.381) (layers F.Cu B.Cu) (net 10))
 (via (at 135.89 95.5675) (size 0.635) (drill 0.381) (layers F.Cu B.Cu) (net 10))
 (via (at 136.8425 91.7575) (size 0.635) (drill 0.381) (layers F.Cu B.Cu) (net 10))
 (via (at 135.89 91.7575) (size 0.635) (drill 0.381) (layers F.Cu B.Cu) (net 10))
 (via (at 134.9375 91.7575) (size 0.635) (drill 0.381) (layers F.Cu B.Cu) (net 10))
 (via (at 133.985 91.7575) (size 0.635) (drill 0.381) (layers F.Cu B.Cu) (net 10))
 (via (at 133.0325 91.7575) (size 0.635) (drill 0.381) (layers F.Cu B.Cu) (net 10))
 (segment (start 144.0725 95.5675) (end 145.0975 96.5925) (width 0.381) (layer F.Cu) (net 8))
 (segment (start 142.8175 95.5675) (end 144.0725 95.5675) (width 0.381) (layer F.Cu) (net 8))
 (segment (start 152.335 95.5675) (end 152.335 96.8375) (width 0.381) (layer F.Cu) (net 4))
 (segment (start 147.4775 96.8375) (end 152.8775 96.8375) (width 0.381) (layer F.Cu) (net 4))
 (segment (start 142.875 93.0275) (end 142.875 93.0275) (width 0.381) (layer B.Cu) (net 3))
 (via (at 142.875 93.0275) (size 0.635) (drill 0.381) (layers F.Cu B.Cu) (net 3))
 (segment (start 142.8175 94.2975) (end 142.8175 93.72) (width 0.381) (layer F.Cu) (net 3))
 (segment (start 142.875 93.6625) (end 142.875 93.0275) (width 0.381) (layer F.Cu) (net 3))
 (segment (start 142.8175 93.72) (end 142.875 93.6625) (width 0.381) (layer F.Cu) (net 3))
 (segment (start 142.875 95.105) (end 142.875 93.0275) (width 0.381) (layer B.Cu) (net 3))
 (segment (start 144.78 93.0275) (end 142.875 93.0275) (width 0.381) (layer B.Cu) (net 3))
 (segment (start 152.85375 91.79375) (end 146.01375 91.79375) (width 0.381) (layer B.Cu) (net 3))
 (segment (start 152.89 91.7575) (end 152.85375 91.79375) (width 0.381) (layer B.Cu) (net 3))
 (segment (start 155.92875 91.79375) (end 158.4325 94.2975) (width 0.381) (layer B.Cu) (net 3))
 (segment (start 152.89 91.7575) (end 152.92625 91.79375) (width 0.381) (layer B.Cu) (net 3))
 (segment (start 146.01375 91.79375) (end 144.78 93.0275) (width 0.381) (layer B.Cu) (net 3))
 (segment (start 152.92625 91.79375) (end 155.92875 91.79375) (width 0.381) (layer B.Cu) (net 3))
 (segment (start 152.92625 91.79375) (end 152.92625 91.79375) (width 0.381) (layer B.Cu) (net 3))
 (via (at 152.92625 91.79375) (size 0.635) (drill 0.381) (layers F.Cu B.Cu) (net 3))
 (segment (start 152.8775 91.77) (end 152.89 91.7575) (width 0.381) (layer F.Cu) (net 3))
 (segment (start 152.8775 94.2975) (end 152.8775 91.77) (width 0.381) (layer F.Cu) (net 3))
 (segment (start 152.8775 94.2975) (end 154.6225 94.2975) (width 0.381) (layer F.Cu) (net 3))
 (segment (start 155.2575 94.9325) (end 155.2575 96.0575) (width 0.381) (layer F.Cu) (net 3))
 (segment (start 154.6225 94.2975) (end 155.2575 94.9325) (width 0.381) (layer F.Cu) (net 3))
 (segment (start 152.8775 100.245) (end 152.9625 100.33) (width 0.381) (layer F.Cu) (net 5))
 (segment (start 152.8775 98.1075) (end 152.8775 100.245) (width 0.381) (layer F.Cu) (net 5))
 (segment (start 155.2575 98.1075) (end 152.8775 98.1075) (width 0.381) (layer F.Cu) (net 5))
 (segment (start 152.9625 100.33) (end 149.5425 100.33) (width 0.381) (layer F.Cu) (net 5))
 (segment (start 149.5425 92.075) (end 149.5425 89.8525) (width 0.381) (layer F.Cu) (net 6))
 (segment (start 146.1225 95.5675) (end 145.0975 94.5425) (width 0.381) (layer F.Cu) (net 6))
 (segment (start 147.4775 95.5675) (end 146.1225 95.5675) (width 0.381) (layer F.Cu) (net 6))
 (segment (start 147.4775 95.5675) (end 148.9075 95.5675) (width 0.381) (layer F.Cu) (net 6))
 (segment (start 149.5425 94.9325) (end 149.5425 92.075) (width 0.381) (layer F.Cu) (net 6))
 (segment (start 148.9075 95.5675) (end 149.5425 94.9325) (width 0.381) (layer F.Cu) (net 6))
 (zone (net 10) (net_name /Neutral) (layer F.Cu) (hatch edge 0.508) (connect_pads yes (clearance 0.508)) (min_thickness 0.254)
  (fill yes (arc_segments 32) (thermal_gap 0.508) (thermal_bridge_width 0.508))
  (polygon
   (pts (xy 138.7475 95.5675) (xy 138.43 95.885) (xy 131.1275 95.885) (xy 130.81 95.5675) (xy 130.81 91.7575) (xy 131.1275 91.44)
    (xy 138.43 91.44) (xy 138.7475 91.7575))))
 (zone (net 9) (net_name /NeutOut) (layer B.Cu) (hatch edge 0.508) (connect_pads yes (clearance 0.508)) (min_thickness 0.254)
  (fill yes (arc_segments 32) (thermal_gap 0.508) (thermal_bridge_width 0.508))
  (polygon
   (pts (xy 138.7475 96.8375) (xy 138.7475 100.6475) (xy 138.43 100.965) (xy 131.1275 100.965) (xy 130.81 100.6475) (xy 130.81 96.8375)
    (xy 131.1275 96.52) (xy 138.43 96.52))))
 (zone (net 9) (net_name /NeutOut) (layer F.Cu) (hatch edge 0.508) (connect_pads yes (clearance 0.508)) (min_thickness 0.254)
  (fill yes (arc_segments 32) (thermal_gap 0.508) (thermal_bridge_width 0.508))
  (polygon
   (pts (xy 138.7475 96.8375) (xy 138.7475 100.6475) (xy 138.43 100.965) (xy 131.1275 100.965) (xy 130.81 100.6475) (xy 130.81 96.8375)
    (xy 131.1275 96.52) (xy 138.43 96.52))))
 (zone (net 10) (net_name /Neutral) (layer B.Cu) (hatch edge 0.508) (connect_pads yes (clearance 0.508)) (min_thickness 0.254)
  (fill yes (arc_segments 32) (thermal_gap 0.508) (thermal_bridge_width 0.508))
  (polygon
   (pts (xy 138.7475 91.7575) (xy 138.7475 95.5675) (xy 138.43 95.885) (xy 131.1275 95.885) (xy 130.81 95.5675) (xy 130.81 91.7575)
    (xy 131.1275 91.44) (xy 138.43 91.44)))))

